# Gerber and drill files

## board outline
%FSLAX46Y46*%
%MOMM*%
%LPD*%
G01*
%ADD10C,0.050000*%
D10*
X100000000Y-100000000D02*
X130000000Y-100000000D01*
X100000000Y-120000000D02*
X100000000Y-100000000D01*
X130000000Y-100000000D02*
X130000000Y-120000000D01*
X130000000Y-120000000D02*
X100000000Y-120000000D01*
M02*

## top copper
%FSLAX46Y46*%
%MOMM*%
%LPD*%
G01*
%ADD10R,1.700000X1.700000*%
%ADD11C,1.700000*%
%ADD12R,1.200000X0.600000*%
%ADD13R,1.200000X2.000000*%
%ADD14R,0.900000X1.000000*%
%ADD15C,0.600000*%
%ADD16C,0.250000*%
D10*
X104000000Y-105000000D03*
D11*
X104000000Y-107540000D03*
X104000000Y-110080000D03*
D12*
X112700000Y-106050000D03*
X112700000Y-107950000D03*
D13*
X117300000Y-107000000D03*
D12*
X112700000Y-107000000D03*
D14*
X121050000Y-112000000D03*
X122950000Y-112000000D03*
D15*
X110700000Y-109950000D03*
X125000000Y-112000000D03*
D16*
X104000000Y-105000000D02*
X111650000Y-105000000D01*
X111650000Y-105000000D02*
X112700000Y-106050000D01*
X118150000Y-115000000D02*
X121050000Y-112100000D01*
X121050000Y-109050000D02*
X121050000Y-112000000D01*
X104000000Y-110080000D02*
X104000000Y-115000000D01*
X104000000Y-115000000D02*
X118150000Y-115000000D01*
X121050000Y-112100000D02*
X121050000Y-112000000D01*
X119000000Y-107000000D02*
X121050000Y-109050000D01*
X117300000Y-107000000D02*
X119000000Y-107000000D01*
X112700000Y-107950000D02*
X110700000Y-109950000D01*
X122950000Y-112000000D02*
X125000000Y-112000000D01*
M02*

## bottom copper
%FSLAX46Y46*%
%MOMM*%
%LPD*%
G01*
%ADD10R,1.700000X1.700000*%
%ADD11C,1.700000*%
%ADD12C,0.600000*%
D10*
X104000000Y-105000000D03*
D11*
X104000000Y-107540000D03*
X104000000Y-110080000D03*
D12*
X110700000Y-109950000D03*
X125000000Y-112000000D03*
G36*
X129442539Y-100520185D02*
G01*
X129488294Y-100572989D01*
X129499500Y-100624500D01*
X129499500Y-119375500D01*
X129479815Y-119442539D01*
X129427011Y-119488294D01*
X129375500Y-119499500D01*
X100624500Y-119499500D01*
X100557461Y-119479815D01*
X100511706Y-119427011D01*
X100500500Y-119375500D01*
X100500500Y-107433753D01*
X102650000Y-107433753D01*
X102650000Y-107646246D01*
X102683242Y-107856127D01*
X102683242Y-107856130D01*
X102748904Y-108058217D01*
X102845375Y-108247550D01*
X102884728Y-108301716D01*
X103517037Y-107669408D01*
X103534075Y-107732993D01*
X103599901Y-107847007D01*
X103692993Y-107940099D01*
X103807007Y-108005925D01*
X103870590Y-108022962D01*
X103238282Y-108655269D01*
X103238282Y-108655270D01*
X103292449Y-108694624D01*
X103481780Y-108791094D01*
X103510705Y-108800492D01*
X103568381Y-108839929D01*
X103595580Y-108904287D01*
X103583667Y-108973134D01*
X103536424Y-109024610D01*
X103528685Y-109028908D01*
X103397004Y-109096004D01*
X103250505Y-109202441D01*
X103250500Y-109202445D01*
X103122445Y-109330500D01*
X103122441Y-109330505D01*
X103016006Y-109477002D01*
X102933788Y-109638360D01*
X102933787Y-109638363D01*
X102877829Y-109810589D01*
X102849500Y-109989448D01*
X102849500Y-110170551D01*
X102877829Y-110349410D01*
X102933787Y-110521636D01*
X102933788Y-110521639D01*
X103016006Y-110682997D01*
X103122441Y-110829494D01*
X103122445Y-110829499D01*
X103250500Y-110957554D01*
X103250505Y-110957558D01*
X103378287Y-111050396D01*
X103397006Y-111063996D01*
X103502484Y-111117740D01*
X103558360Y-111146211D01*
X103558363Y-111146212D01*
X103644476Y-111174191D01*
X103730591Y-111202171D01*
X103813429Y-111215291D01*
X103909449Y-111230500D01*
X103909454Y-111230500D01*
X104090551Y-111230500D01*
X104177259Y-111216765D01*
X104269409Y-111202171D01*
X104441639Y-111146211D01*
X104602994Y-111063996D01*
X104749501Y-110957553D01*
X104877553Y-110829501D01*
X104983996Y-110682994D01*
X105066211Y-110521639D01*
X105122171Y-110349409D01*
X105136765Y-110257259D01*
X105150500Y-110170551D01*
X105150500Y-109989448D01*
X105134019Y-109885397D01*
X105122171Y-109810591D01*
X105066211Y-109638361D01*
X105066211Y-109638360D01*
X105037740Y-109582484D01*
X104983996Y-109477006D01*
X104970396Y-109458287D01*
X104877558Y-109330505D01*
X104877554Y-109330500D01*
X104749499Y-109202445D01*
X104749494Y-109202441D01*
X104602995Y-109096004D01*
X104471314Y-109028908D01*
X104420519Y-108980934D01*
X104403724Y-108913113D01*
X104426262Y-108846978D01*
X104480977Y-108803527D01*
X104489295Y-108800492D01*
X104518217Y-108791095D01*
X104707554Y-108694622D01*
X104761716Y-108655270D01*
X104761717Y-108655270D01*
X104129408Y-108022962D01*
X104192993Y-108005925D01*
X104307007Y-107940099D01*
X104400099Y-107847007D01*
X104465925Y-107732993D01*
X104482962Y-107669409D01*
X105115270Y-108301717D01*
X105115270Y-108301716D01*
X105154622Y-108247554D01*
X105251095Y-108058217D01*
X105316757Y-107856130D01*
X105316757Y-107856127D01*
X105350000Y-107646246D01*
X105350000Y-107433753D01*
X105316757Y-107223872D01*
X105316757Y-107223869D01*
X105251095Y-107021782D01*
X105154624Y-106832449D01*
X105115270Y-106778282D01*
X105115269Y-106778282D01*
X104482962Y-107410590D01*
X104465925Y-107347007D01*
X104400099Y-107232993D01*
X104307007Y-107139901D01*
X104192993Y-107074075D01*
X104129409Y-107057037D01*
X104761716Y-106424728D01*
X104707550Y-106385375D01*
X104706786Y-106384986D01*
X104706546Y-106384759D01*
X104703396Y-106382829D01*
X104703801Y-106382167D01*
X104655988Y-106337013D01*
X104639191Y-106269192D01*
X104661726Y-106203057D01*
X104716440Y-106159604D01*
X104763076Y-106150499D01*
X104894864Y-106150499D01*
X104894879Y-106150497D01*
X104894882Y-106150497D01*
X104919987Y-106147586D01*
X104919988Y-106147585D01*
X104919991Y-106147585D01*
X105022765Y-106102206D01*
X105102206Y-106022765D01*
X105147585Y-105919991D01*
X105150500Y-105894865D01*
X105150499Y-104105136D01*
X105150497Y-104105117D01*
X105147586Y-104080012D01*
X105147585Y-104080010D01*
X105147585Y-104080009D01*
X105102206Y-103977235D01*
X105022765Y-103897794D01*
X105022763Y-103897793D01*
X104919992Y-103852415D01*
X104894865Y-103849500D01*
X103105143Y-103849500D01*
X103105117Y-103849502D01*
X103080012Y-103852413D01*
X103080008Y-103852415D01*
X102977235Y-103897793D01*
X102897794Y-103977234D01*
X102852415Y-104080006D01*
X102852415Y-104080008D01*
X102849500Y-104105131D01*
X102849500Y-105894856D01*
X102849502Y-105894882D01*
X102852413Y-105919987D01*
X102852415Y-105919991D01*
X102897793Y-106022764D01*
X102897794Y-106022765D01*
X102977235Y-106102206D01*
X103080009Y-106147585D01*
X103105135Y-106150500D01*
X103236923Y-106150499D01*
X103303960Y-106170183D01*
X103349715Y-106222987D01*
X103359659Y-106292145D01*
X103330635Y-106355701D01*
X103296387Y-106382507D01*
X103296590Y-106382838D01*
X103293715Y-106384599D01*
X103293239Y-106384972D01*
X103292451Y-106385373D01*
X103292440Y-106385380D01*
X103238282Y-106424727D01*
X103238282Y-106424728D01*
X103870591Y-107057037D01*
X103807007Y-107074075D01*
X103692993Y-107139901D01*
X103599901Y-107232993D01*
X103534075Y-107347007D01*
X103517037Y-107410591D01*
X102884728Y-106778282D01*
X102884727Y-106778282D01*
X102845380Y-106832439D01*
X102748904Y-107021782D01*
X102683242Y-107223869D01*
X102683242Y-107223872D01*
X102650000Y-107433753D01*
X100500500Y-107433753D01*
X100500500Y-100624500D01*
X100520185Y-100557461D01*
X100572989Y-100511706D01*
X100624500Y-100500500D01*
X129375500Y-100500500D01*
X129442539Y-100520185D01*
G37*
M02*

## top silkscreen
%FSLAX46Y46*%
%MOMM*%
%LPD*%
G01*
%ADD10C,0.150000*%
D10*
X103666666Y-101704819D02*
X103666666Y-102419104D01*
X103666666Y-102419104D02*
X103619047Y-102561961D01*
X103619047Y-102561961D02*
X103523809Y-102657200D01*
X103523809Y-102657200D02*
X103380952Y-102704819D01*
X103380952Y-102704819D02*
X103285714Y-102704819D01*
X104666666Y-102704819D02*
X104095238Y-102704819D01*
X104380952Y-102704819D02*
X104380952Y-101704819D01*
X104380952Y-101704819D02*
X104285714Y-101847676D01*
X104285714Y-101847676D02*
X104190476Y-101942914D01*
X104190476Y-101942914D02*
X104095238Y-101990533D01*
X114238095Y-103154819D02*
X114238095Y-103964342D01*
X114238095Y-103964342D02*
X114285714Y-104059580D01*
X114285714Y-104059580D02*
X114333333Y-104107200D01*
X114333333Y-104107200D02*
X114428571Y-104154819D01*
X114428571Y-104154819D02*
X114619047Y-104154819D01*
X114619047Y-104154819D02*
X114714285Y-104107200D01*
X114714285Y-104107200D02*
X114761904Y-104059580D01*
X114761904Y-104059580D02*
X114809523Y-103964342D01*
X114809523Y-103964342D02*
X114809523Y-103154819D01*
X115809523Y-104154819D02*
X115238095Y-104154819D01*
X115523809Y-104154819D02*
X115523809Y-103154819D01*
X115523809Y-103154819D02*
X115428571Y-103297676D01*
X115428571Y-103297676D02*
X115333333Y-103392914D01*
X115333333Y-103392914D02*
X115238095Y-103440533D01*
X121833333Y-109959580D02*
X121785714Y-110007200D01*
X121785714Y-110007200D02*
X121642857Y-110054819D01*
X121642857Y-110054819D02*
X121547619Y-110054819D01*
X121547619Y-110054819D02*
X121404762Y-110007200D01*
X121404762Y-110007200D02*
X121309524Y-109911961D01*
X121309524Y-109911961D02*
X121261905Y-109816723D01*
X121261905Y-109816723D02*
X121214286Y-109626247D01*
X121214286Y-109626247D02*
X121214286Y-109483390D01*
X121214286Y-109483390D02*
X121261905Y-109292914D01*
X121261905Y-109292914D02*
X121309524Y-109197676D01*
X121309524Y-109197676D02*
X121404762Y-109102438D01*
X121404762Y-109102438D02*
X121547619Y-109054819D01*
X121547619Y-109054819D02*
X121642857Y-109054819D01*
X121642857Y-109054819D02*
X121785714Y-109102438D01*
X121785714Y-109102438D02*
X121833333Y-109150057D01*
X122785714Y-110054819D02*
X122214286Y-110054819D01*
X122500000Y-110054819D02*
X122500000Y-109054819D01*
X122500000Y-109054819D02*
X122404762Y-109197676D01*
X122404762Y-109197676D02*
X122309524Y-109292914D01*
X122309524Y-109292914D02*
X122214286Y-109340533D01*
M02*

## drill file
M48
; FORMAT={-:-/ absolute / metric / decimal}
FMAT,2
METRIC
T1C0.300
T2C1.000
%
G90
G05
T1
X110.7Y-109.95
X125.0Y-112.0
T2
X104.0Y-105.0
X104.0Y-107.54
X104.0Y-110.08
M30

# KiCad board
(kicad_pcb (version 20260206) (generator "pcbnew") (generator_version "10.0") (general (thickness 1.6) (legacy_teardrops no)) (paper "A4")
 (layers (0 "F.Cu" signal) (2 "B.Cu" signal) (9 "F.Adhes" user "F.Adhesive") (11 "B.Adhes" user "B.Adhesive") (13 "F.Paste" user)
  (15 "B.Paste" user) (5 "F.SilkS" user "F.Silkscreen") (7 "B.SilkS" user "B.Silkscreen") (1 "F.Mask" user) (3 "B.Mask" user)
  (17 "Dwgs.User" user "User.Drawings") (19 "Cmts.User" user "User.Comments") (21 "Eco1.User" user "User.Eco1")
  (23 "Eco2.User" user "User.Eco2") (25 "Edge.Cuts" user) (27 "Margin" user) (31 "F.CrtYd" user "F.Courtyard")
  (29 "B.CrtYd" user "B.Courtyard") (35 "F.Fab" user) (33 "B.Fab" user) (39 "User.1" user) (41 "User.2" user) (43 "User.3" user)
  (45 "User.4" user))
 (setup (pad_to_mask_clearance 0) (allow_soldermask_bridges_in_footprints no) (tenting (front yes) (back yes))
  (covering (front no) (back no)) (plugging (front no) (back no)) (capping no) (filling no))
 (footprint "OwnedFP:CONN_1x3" (layer "F.Cu") (at 104 105)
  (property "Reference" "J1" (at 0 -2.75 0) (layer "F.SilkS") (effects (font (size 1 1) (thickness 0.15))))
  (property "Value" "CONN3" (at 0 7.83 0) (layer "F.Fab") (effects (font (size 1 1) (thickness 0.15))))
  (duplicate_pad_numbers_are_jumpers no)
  (pad "1" thru_hole rect (at 0 0) (size 1.7 1.7) (drill 1) (layers "*.Cu" "*.Mask") (remove_unused_layers no) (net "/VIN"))
  (pad "2" thru_hole circle (at 0 2.54) (size 1.7 1.7) (drill 1) (layers "*.Cu" "*.Mask") (remove_unused_layers no) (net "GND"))
  (pad "3" thru_hole circle (at 0 5.08) (size 1.7 1.7) (drill 1) (layers "*.Cu" "*.Mask") (remove_unused_layers no) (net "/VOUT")))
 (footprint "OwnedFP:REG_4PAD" (layer "F.Cu") (at 115 107)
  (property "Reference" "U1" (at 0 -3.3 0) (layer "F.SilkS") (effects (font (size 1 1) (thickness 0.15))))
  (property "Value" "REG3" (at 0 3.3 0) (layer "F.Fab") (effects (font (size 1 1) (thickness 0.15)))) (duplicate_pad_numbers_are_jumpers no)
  (pad "1" smd rect (at -2.3 -0.95) (size 1.2 0.6) (layers "F.Cu" "F.Mask" "F.Paste") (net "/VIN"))
  (pad "2" smd rect (at -2.3 0.95) (size 1.2 0.6) (layers "F.Cu" "F.Mask" "F.Paste") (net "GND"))
  (pad "3" smd rect (at 2.3 0) (size 1.2 2) (layers "F.Cu" "F.Mask" "F.Paste") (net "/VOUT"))
  (pad "4" smd rect (at -2.3 0) (size 1.2 0.6) (layers "F.Cu" "F.Mask" "F.Paste") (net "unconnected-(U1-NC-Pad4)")))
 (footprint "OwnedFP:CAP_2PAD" (layer "F.Cu") (at 122 112)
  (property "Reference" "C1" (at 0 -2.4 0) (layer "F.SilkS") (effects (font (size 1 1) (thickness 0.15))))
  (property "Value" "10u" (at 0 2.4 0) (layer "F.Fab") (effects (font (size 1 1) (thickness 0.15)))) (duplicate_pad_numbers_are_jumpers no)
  (pad "1" smd rect (at -0.95 0) (size 0.9 1) (layers "F.Cu" "F.Mask" "F.Paste") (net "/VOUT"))
  (pad "2" smd rect (at 0.95 0) (size 0.9 1) (layers "F.Cu" "F.Mask" "F.Paste") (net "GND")))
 (gr_line (start 100 100) (end 130 100) (stroke (width 0.05) (type default)) (layer "Edge.Cuts"))
 (gr_line (start 100 120) (end 100 100) (stroke (width 0.05) (type default)) (layer "Edge.Cuts"))
 (gr_line (start 130 100) (end 130 120) (stroke (width 0.05) (type default)) (layer "Edge.Cuts"))
 (gr_line (start 130 120) (end 100 120) (stroke (width 0.05) (type default)) (layer "Edge.Cuts"))
 (segment (start 104 105) (end 111.65 105) (width 0.25) (layer "F.Cu") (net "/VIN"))
 (segment (start 111.65 105) (end 112.7 106.05) (width 0.25) (layer "F.Cu") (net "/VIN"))
 (segment (start 118.15 115) (end 121.05 112.1) (width 0.25) (layer "F.Cu") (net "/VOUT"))
 (segment (start 121.05 109.05) (end 121.05 112) (width 0.25) (layer "F.Cu") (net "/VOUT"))
 (segment (start 104 110.08) (end 104 115) (width 0.25) (layer "F.Cu") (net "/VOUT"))
 (segment (start 104 115) (end 118.15 115) (width 0.25) (layer "F.Cu") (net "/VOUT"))
 (segment (start 121.05 112.1) (end 121.05 112) (width 0.25) (layer "F.Cu") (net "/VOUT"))
 (segment (start 119 107) (end 121.05 109.05) (width 0.25) (layer "F.Cu") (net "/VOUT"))
 (segment (start 117.3 107) (end 119 107) (width 0.25) (layer "F.Cu") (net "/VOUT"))
 (segment (start 112.7 107.95) (end 110.7 109.95) (width 0.25) (layer "F.Cu") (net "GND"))
 (segment (start 122.95 112) (end 125 112) (width 0.25) (layer "F.Cu") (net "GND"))
 (via (at 110.7 109.95) (size 0.6) (drill 0.3) (layers "F.Cu" "B.Cu") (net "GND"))
 (via (at 125 112) (size 0.6) (drill 0.3) (layers "F.Cu" "B.Cu") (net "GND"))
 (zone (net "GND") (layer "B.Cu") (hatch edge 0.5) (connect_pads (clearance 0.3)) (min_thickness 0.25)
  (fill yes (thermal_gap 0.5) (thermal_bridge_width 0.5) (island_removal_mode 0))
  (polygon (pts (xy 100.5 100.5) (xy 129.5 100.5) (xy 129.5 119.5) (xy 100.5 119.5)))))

